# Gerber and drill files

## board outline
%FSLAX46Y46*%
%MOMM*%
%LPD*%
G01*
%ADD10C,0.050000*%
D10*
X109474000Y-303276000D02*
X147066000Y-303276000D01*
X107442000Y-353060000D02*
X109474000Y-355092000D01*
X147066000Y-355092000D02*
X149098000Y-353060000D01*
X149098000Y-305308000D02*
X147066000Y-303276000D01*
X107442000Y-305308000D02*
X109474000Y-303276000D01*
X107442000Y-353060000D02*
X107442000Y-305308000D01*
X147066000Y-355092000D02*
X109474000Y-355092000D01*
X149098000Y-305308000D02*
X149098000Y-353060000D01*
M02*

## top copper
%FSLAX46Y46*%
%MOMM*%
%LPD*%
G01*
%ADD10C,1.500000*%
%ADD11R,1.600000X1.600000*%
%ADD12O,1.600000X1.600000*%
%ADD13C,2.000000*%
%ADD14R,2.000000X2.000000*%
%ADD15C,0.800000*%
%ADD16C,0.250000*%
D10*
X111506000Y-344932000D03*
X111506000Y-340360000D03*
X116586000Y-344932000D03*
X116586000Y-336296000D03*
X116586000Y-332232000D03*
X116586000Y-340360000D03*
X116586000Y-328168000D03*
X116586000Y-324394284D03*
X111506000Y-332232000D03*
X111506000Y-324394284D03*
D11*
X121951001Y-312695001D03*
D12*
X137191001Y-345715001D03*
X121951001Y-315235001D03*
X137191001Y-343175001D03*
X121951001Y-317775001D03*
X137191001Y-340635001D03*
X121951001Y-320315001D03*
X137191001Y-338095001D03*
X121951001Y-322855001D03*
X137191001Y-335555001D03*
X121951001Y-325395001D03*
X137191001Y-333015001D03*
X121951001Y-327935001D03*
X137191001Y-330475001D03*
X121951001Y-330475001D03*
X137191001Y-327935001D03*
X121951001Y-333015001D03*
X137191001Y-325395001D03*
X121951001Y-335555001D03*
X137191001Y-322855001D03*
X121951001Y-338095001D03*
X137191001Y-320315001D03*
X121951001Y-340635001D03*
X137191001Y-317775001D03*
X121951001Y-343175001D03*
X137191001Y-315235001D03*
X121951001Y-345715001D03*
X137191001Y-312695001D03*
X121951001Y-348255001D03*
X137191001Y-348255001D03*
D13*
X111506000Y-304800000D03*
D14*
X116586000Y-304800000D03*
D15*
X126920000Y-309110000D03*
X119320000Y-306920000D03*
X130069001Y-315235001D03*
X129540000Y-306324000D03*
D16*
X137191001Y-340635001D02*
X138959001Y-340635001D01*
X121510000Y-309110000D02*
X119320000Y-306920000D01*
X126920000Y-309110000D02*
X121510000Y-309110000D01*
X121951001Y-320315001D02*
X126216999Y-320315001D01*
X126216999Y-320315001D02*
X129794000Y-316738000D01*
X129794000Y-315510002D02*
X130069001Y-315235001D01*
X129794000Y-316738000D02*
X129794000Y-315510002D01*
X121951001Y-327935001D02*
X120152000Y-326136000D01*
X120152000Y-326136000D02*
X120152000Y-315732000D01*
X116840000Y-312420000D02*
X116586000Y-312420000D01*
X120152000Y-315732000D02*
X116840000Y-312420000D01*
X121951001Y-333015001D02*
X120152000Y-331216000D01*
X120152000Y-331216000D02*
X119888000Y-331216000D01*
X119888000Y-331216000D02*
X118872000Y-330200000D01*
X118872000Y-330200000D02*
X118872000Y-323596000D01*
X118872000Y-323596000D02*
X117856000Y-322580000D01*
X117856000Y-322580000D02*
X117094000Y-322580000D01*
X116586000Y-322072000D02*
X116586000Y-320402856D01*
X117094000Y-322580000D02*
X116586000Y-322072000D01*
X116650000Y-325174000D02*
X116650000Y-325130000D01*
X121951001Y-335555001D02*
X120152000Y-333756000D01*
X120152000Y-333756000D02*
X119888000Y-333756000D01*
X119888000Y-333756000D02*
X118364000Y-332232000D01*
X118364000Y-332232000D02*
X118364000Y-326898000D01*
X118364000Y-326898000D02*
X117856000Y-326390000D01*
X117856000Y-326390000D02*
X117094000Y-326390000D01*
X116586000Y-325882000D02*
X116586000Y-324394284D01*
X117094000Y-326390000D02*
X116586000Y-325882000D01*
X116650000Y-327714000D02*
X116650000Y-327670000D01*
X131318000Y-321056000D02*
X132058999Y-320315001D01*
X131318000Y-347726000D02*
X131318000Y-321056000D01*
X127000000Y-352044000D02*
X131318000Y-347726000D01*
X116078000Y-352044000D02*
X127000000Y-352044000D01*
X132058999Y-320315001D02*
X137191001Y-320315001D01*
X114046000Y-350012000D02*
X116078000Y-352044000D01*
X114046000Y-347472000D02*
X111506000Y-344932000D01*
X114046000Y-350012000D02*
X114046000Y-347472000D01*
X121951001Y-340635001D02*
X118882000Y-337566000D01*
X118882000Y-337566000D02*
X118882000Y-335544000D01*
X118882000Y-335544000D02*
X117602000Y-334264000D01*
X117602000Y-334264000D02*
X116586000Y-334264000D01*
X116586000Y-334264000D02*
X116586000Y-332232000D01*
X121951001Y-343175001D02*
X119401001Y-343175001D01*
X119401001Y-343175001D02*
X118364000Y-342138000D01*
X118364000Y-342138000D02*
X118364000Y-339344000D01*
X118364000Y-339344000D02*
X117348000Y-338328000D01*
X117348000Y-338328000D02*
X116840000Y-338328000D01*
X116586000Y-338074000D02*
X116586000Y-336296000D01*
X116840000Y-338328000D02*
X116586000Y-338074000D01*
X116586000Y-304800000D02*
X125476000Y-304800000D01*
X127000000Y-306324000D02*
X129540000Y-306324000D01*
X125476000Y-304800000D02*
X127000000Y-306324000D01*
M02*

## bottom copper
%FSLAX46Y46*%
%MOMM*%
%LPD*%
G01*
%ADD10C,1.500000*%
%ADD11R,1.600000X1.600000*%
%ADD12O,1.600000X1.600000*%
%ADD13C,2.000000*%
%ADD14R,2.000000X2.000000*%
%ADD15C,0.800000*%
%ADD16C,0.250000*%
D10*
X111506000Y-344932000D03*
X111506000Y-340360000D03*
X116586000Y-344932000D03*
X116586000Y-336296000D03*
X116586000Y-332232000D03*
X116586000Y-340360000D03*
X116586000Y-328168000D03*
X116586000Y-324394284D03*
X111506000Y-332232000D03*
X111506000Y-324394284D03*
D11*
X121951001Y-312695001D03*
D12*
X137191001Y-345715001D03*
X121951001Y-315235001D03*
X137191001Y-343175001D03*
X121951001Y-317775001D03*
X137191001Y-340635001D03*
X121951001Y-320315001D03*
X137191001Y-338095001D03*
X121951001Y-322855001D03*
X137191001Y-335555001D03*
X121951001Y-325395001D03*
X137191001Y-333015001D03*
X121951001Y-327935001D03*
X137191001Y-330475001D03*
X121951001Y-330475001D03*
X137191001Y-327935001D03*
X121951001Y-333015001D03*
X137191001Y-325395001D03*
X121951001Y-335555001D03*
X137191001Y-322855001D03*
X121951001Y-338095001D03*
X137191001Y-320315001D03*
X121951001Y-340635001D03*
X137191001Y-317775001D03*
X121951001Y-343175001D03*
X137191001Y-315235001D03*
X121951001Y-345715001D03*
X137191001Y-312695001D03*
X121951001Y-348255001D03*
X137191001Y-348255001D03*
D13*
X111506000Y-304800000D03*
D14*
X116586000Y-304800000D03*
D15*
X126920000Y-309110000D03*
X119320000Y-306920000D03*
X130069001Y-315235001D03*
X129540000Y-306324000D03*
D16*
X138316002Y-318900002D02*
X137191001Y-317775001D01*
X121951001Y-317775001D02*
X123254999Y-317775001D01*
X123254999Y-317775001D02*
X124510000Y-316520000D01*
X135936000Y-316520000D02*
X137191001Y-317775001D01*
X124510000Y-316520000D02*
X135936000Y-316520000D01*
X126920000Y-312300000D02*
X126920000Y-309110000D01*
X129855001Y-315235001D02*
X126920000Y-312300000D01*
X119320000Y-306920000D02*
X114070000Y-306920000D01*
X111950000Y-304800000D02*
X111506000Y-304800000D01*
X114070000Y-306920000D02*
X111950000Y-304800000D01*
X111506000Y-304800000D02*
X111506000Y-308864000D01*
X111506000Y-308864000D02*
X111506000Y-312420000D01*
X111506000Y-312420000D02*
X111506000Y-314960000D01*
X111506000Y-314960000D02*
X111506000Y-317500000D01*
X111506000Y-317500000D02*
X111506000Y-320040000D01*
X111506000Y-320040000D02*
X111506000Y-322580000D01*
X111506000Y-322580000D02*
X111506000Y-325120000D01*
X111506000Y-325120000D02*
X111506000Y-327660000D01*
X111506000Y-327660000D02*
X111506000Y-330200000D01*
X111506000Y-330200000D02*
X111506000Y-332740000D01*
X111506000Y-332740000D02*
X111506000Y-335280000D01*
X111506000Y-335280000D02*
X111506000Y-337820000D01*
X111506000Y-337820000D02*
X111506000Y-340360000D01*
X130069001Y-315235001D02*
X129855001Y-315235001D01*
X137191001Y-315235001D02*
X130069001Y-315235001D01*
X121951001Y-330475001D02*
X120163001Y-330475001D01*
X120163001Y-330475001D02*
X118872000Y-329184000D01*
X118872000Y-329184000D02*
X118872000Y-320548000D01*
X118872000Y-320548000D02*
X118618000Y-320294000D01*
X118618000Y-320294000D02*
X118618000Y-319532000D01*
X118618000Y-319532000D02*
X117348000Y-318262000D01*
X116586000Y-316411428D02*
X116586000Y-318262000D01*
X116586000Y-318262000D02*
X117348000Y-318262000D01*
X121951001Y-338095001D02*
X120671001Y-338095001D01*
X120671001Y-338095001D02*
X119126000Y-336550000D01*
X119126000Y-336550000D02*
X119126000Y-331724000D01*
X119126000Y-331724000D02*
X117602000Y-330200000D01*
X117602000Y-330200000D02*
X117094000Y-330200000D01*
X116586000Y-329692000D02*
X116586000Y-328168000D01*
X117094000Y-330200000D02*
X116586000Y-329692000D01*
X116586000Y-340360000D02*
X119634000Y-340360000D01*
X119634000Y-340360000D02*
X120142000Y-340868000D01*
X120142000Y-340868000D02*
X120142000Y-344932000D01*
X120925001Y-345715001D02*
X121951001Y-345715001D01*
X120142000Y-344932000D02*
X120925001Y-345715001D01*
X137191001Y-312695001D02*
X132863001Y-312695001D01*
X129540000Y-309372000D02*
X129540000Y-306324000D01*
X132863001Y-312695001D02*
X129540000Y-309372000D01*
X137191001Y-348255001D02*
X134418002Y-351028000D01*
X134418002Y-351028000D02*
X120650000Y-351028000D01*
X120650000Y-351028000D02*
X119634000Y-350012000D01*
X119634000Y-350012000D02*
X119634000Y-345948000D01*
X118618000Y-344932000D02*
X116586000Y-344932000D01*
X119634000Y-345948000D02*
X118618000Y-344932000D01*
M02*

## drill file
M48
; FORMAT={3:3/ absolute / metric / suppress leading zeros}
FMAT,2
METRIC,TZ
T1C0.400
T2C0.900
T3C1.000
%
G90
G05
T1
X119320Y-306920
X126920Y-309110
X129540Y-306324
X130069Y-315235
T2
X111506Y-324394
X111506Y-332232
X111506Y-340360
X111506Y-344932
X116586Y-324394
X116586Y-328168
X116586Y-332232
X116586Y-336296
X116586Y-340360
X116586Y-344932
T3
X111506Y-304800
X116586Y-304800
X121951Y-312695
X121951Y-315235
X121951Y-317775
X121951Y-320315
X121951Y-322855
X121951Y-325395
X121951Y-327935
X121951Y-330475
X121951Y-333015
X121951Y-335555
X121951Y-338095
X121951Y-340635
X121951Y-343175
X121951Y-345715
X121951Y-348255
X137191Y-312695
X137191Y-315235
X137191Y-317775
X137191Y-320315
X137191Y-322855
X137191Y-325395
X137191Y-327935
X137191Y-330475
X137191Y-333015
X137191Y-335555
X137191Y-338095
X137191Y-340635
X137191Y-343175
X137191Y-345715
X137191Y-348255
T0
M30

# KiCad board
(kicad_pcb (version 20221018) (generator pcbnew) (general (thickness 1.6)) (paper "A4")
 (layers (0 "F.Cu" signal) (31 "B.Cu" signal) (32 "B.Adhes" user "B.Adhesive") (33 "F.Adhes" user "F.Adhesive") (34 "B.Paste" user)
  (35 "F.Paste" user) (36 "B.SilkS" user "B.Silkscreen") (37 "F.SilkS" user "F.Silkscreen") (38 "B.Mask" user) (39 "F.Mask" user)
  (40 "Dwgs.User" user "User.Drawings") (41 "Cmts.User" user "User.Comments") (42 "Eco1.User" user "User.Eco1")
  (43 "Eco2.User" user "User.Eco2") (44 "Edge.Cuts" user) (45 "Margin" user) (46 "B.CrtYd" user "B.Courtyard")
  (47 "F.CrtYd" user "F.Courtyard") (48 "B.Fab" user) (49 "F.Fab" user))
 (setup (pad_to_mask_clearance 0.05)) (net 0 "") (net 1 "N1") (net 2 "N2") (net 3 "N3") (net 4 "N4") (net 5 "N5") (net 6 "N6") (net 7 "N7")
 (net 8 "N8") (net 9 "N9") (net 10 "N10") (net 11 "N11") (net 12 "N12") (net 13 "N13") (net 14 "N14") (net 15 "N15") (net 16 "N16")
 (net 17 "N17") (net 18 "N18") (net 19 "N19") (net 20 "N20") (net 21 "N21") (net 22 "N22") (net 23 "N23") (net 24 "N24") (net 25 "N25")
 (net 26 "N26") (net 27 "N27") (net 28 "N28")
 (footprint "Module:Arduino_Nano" (layer "F.Cu") (at 121.951001 312.695001)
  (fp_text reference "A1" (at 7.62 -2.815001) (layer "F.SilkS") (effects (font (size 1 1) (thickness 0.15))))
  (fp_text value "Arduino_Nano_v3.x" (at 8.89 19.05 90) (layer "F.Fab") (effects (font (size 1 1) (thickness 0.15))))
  (pad "1" thru_hole rect (at 0 0) (size 1.6 1.6) (drill 1) (layers "*.Cu" "*.Mask") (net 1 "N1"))
  (pad "2" thru_hole oval (at 0 2.54) (size 1.6 1.6) (drill 1) (layers "*.Cu" "*.Mask") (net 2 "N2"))
  (pad "3" thru_hole oval (at 0 5.08) (size 1.6 1.6) (drill 1) (layers "*.Cu" "*.Mask") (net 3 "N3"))
  (pad "4" thru_hole oval (at 0 7.62) (size 1.6 1.6) (drill 1) (layers "*.Cu" "*.Mask") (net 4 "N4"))
  (pad "5" thru_hole oval (at 0 10.16) (size 1.6 1.6) (drill 1) (layers "*.Cu" "*.Mask") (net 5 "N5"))
  (pad "6" thru_hole oval (at 0 12.7) (size 1.6 1.6) (drill 1) (layers "*.Cu" "*.Mask") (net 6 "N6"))
  (pad "7" thru_hole oval (at 0 15.24) (size 1.6 1.6) (drill 1) (layers "*.Cu" "*.Mask") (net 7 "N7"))
  (pad "8" thru_hole oval (at 0 17.78) (size 1.6 1.6) (drill 1) (layers "*.Cu" "*.Mask") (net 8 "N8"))
  (pad "9" thru_hole oval (at 0 20.32) (size 1.6 1.6) (drill 1) (layers "*.Cu" "*.Mask") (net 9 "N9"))
  (pad "10" thru_hole oval (at 0 22.86) (size 1.6 1.6) (drill 1) (layers "*.Cu" "*.Mask") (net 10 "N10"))
  (pad "11" thru_hole oval (at 0 25.4) (size 1.6 1.6) (drill 1) (layers "*.Cu" "*.Mask") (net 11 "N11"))
  (pad "12" thru_hole oval (at 0 27.94) (size 1.6 1.6) (drill 1) (layers "*.Cu" "*.Mask") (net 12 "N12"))
  (pad "13" thru_hole oval (at 0 30.48) (size 1.6 1.6) (drill 1) (layers "*.Cu" "*.Mask") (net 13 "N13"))
  (pad "14" thru_hole oval (at 0 33.02) (size 1.6 1.6) (drill 1) (layers "*.Cu" "*.Mask") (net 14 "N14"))
  (pad "15" thru_hole oval (at 0 35.56) (size 1.6 1.6) (drill 1) (layers "*.Cu" "*.Mask") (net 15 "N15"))
  (pad "16" thru_hole oval (at 15.24 35.56) (size 1.6 1.6) (drill 1) (layers "*.Cu" "*.Mask") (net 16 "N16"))
  (pad "17" thru_hole oval (at 15.24 33.02) (size 1.6 1.6) (drill 1) (layers "*.Cu" "*.Mask") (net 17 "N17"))
  (pad "18" thru_hole oval (at 15.24 30.48) (size 1.6 1.6) (drill 1) (layers "*.Cu" "*.Mask") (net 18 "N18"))
  (pad "19" thru_hole oval (at 15.24 27.94) (size 1.6 1.6) (drill 1) (layers "*.Cu" "*.Mask") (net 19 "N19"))
  (pad "20" thru_hole oval (at 15.24 25.4) (size 1.6 1.6) (drill 1) (layers "*.Cu" "*.Mask") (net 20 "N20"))
  (pad "21" thru_hole oval (at 15.24 22.86) (size 1.6 1.6) (drill 1) (layers "*.Cu" "*.Mask") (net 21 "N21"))
  (pad "22" thru_hole oval (at 15.24 20.32) (size 1.6 1.6) (drill 1) (layers "*.Cu" "*.Mask") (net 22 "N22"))
  (pad "23" thru_hole oval (at 15.24 17.78) (size 1.6 1.6) (drill 1) (layers "*.Cu" "*.Mask") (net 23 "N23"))
  (pad "24" thru_hole oval (at 15.24 15.24) (size 1.6 1.6) (drill 1) (layers "*.Cu" "*.Mask") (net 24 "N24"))
  (pad "25" thru_hole oval (at 15.24 12.7) (size 1.6 1.6) (drill 1) (layers "*.Cu" "*.Mask") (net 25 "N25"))
  (pad "26" thru_hole oval (at 15.24 10.16) (size 1.6 1.6) (drill 1) (layers "*.Cu" "*.Mask") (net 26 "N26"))
  (pad "27" thru_hole oval (at 15.24 7.62) (size 1.6 1.6) (drill 1) (layers "*.Cu" "*.Mask") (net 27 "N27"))
  (pad "28" thru_hole oval (at 15.24 5.08) (size 1.6 1.6) (drill 1) (layers "*.Cu" "*.Mask") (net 3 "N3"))
  (pad "29" thru_hole oval (at 15.24 2.54) (size 1.6 1.6) (drill 1) (layers "*.Cu" "*.Mask") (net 4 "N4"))
  (pad "30" thru_hole oval (at 15.24 0) (size 1.6 1.6) (drill 1) (layers "*.Cu" "*.Mask") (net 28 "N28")))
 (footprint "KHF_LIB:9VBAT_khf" (layer "F.Cu") (at 111.506 304.8)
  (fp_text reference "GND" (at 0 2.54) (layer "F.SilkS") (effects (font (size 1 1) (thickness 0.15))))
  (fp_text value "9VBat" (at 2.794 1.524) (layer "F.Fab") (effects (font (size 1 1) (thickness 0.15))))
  (pad "1" thru_hole circle (at 0 0) (size 2 2) (drill 1) (layers "*.Cu" "*.Mask") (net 4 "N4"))
  (pad "2" thru_hole rect (at 5.08 0) (size 2 2) (drill 1) (layers "*.Cu" "*.Mask") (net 28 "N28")))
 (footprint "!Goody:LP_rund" (layer "F.Cu") (at 116.586 336.296)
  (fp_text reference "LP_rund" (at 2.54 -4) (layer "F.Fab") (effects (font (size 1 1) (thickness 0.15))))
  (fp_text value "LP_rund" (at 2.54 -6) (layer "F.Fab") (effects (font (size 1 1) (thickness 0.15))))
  (pad "1" thru_hole circle (at 0 0) (size 1.5 1.5) (drill 0.9) (layers "*.Cu" "*.Mask") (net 13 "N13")))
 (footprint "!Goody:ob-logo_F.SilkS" (layer "F.Cu") (at 130.048 329.692 90)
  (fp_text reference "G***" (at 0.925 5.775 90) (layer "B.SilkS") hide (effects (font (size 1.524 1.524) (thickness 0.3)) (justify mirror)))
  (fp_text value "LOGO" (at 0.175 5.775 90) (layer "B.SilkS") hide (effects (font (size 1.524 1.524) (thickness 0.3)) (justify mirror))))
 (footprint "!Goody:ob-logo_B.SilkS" (layer "F.Cu") (at 146.05 323.596 90)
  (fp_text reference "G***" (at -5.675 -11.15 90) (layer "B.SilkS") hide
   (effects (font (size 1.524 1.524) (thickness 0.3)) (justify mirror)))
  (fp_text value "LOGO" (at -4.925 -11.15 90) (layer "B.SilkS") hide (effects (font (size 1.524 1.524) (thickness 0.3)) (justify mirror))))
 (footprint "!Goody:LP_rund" (layer "F.Cu") (at 116.586 344.932)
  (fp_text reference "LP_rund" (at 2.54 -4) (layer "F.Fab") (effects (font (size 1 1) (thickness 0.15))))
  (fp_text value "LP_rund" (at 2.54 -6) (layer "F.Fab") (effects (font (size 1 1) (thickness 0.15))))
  (pad "1" thru_hole circle (at 0 0) (size 1.5 1.5) (drill 0.9) (layers "*.Cu" "*.Mask") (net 16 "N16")))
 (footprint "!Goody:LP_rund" (layer "F.Cu") (at 111.506 340.36)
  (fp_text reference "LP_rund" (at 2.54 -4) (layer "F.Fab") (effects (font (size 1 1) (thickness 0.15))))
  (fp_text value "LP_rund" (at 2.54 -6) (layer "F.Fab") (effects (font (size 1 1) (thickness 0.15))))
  (pad "1" thru_hole circle (at 0 0) (size 1.5 1.5) (drill 0.9) (layers "*.Cu" "*.Mask") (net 4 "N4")))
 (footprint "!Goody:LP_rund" (layer "F.Cu") (at 111.506 344.932)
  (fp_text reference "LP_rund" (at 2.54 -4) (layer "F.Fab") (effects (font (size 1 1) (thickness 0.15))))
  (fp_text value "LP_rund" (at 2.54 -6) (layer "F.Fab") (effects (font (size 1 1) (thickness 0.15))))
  (pad "1" thru_hole circle (at 0 0) (size 1.5 1.5) (drill 0.9) (layers "*.Cu" "*.Mask") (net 27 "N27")))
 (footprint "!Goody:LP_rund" (layer "F.Cu") (at 116.586 324.394284)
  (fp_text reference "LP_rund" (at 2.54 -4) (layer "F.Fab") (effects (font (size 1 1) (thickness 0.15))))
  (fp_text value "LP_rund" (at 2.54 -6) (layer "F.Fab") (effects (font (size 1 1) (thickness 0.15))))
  (pad "1" thru_hole circle (at 0 0) (size 1.5 1.5) (drill 0.9) (layers "*.Cu" "*.Mask") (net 10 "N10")))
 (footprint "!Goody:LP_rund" (layer "F.Cu") (at 111.506 330.2)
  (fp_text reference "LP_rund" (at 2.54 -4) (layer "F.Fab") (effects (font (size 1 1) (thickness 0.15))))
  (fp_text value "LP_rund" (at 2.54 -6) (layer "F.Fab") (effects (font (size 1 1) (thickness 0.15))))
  (pad "1" thru_hole circle (at 0 -5.805716) (size 1.5 1.5) (drill 0.9) (layers "*.Cu" "*.Mask") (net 4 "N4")))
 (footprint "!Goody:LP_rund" (layer "F.Cu") (at 116.586 328.168)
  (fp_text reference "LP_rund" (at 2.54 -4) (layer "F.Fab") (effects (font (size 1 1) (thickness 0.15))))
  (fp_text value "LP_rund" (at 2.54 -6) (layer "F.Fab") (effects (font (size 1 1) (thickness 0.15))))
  (pad "1" thru_hole circle (at 0 0) (size 1.5 1.5) (drill 0.9) (layers "*.Cu" "*.Mask") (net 11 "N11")))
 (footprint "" (layer "F.Cu") (at 112.268 348.488)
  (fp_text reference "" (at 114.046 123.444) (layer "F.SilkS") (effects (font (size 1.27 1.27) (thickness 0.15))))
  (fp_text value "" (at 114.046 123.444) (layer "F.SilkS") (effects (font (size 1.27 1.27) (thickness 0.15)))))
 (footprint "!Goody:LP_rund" (layer "F.Cu") (at 111.506 335.13486)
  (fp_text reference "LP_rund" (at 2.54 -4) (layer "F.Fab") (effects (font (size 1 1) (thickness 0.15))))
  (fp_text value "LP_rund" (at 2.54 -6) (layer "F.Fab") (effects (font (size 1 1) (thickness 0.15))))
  (pad "1" thru_hole circle (at 0 -2.90286) (size 1.5 1.5) (drill 0.9) (layers "*.Cu" "*.Mask") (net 4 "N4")))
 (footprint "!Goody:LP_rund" (layer "F.Cu") (at 116.586 340.36)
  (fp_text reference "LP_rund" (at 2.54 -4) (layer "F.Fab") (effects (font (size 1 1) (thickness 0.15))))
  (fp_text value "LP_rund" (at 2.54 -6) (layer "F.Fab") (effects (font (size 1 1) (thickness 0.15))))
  (pad "1" thru_hole circle (at 0 0) (size 1.5 1.5) (drill 0.9) (layers "*.Cu" "*.Mask") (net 14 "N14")))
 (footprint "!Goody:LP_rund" (layer "F.Cu") (at 116.586 332.232)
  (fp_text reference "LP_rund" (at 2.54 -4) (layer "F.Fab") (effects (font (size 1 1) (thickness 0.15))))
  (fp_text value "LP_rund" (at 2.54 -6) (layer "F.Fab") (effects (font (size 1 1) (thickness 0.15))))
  (pad "1" thru_hole circle (at 0 0) (size 1.5 1.5) (drill 0.9) (layers "*.Cu" "*.Mask") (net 12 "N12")))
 (gr_line (start 107.442 353.06) (end 107.442 305.308) (stroke (width 0.05) (type solid)) (layer "Edge.Cuts"))
 (gr_line (start 109.474 303.276) (end 147.066 303.276) (stroke (width 0.05) (type solid)) (layer "Edge.Cuts"))
 (gr_line (start 107.442 305.308) (end 109.474 303.276) (stroke (width 0.05) (type solid)) (layer "Edge.Cuts"))
 (gr_line (start 147.066 355.092) (end 149.098 353.06) (stroke (width 0.05) (type solid)) (layer "Edge.Cuts"))
 (gr_line (start 147.066 355.092) (end 109.474 355.092) (stroke (width 0.05) (type solid)) (layer "Edge.Cuts"))
 (gr_line (start 149.098 305.308) (end 147.066 303.276) (stroke (width 0.05) (type solid)) (layer "Edge.Cuts"))
 (gr_line (start 149.098 305.308) (end 149.098 353.06) (stroke (width 0.05) (type solid)) (layer "Edge.Cuts"))
 (gr_line (start 107.442 353.06) (end 109.474 355.092) (stroke (width 0.05) (type solid)) (layer "Edge.Cuts"))
 (segment (start 138.316002 318.900002) (end 137.191001 317.775001) (width 0.25) (layer "B.Cu") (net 3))
 (segment (start 121.951001 317.775001) (end 123.254999 317.775001) (width 0.25) (layer "B.Cu") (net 3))
 (segment (start 135.936 316.52) (end 137.191001 317.775001) (width 0.25) (layer "B.Cu") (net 3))
 (segment (start 123.254999 317.775001) (end 124.51 316.52) (width 0.25) (layer "B.Cu") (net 3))
 (segment (start 124.51 316.52) (end 135.936 316.52) (width 0.25) (layer "B.Cu") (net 3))
 (segment (start 137.191001 340.635001) (end 138.959001 340.635001) (width 0.25) (layer "F.Cu") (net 19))
 (segment (start 129.794 315.510002) (end 130.069001 315.235001) (width 0.25) (layer "F.Cu") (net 4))
 (segment (start 121.51 309.11) (end 119.32 306.92) (width 0.25) (layer "F.Cu") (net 4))
 (segment (start 129.794 316.738) (end 129.794 315.510002) (width 0.25) (layer "F.Cu") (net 4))
 (segment (start 126.216999 320.315001) (end 129.794 316.738) (width 0.25) (layer "F.Cu") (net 4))
 (segment (start 126.92 309.11) (end 121.51 309.11) (width 0.25) (layer "F.Cu") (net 4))
 (segment (start 121.951001 320.315001) (end 126.216999 320.315001) (width 0.25) (layer "F.Cu") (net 4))
 (via (at 126.92 309.11) (size 0.8) (drill 0.4) (layers "F.Cu" "B.Cu") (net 4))
 (via (at 130.069001 315.235001) (size 0.8) (drill 0.4) (layers "F.Cu" "B.Cu") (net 4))
 (via (at 119.32 306.92) (size 0.8) (drill 0.4) (layers "F.Cu" "B.Cu") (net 4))
 (segment (start 111.95 304.8) (end 111.506 304.8) (width 0.25) (layer "B.Cu") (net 4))
 (segment (start 111.506 330.2) (end 111.506 332.74) (width 0.25) (layer "B.Cu") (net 4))
 (segment (start 111.506 325.12) (end 111.506 327.66) (width 0.25) (layer "B.Cu") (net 4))
 (segment (start 111.506 312.42) (end 111.506 314.96) (width 0.25) (layer "B.Cu") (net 4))
 (segment (start 111.506 335.28) (end 111.506 337.82) (width 0.25) (layer "B.Cu") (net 4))
 (segment (start 111.506 332.74) (end 111.506 335.28) (width 0.25) (layer "B.Cu") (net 4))
 (segment (start 111.506 327.66) (end 111.506 330.2) (width 0.25) (layer "B.Cu") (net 4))
 (segment (start 137.191001 315.235001) (end 130.069001 315.235001) (width 0.25) (layer "B.Cu") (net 4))
 (segment (start 111.506 308.864) (end 111.506 312.42) (width 0.25) (layer "B.Cu") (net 4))
 (segment (start 111.506 320.04) (end 111.506 322.58) (width 0.25) (layer "B.Cu") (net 4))
 (segment (start 130.069001 315.235001) (end 129.855001 315.235001) (width 0.25) (layer "B.Cu") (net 4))
 (segment (start 111.506 337.82) (end 111.506 340.36) (width 0.25) (layer "B.Cu") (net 4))
 (segment (start 111.506 304.8) (end 111.506 308.864) (width 0.25) (layer "B.Cu") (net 4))
 (segment (start 111.506 322.58) (end 111.506 325.12) (width 0.25) (layer "B.Cu") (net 4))
 (segment (start 114.07 306.92) (end 111.95 304.8) (width 0.25) (layer "B.Cu") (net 4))
 (segment (start 119.32 306.92) (end 114.07 306.92) (width 0.25) (layer "B.Cu") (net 4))
 (segment (start 126.92 312.3) (end 126.92 309.11) (width 0.25) (layer "B.Cu") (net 4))
 (segment (start 111.506 314.96) (end 111.506 317.5) (width 0.25) (layer "B.Cu") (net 4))
 (segment (start 111.506 317.5) (end 111.506 320.04) (width 0.25) (layer "B.Cu") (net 4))
 (segment (start 129.855001 315.235001) (end 126.92 312.3) (width 0.25) (layer "B.Cu") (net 4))
 (segment (start 120.152 326.136) (end 120.152 315.732) (width 0.25) (layer "F.Cu") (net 7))
 (segment (start 121.951001 327.935001) (end 120.152 326.136) (width 0.25) (layer "F.Cu") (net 7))
 (segment (start 120.152 315.732) (end 116.84 312.42) (width 0.25) (layer "F.Cu") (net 7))
 (segment (start 116.84 312.42) (end 116.586 312.42) (width 0.25) (layer "F.Cu") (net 7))
 (segment (start 118.618 319.532) (end 117.348 318.262) (width 0.25) (layer "B.Cu") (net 8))
 (segment (start 118.872 329.184) (end 118.872 320.548) (width 0.25) (layer "B.Cu") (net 8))
 (segment (start 121.951001 330.475001) (end 120.163001 330.475001) (width 0.25) (layer "B.Cu") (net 8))
 (segment (start 120.163001 330.475001) (end 118.872 329.184) (width 0.25) (layer "B.Cu") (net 8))
 (segment (start 116.586 316.411428) (end 116.586 318.262) (width 0.25) (layer "B.Cu") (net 8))
 (segment (start 116.586 318.262) (end 117.348 318.262) (width 0.25) (layer "B.Cu") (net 8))
 (segment (start 118.618 320.294) (end 118.618 319.532) (width 0.25) (layer "B.Cu") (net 8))
 (segment (start 118.872 320.548) (end 118.618 320.294) (width 0.25) (layer "B.Cu") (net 8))
 (segment (start 119.888 331.216) (end 118.872 330.2) (width 0.25) (layer "F.Cu") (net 9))
 (segment (start 117.856 322.58) (end 117.094 322.58) (width 0.25) (layer "F.Cu") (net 9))
 (segment (start 118.872 323.596) (end 117.856 322.58) (width 0.25) (layer "F.Cu") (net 9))
 (segment (start 118.872 330.2) (end 118.872 323.596) (width 0.25) (layer "F.Cu") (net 9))
 (segment (start 117.094 322.58) (end 116.586 322.072) (width 0.25) (layer "F.Cu") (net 9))
 (segment (start 120.152 331.216) (end 119.888 331.216) (width 0.25) (layer "F.Cu") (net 9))
 (segment (start 116.586 322.072) (end 116.586 320.402856) (width 0.25) (layer "F.Cu") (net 9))
 (segment (start 121.951001 333.015001) (end 120.152 331.216) (width 0.25) (layer "F.Cu") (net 9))
 (segment (start 120.152 333.756) (end 119.888 333.756) (width 0.25) (layer "F.Cu") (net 10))
 (segment (start 118.364 332.232) (end 118.364 326.898) (width 0.25) (layer "F.Cu") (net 10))
 (segment (start 117.856 326.39) (end 117.094 326.39) (width 0.25) (layer "F.Cu") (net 10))
 (segment (start 121.951001 335.555001) (end 120.152 333.756) (width 0.25) (layer "F.Cu") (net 10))
 (segment (start 119.888 333.756) (end 118.364 332.232) (width 0.25) (layer "F.Cu") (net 10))
 (segment (start 116.65 325.174) (end 116.65 325.13) (width 0.25) (layer "F.Cu") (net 10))
 (segment (start 117.094 326.39) (end 116.586 325.882) (width 0.25) (layer "F.Cu") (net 10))
 (segment (start 118.364 326.898) (end 117.856 326.39) (width 0.25) (layer "F.Cu") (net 10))
 (segment (start 116.586 325.882) (end 116.586 324.394284) (width 0.25) (layer "F.Cu") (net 10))
 (segment (start 116.65 327.714) (end 116.65 327.67) (width 0.25) (layer "F.Cu") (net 11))
 (segment (start 121.951001 338.095001) (end 120.671001 338.095001) (width 0.25) (layer "B.Cu") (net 11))
 (segment (start 119.126 336.55) (end 119.126 331.724) (width 0.25) (layer "B.Cu") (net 11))
 (segment (start 116.586 329.692) (end 116.586 328.168) (width 0.25) (layer "B.Cu") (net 11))
 (segment (start 117.094 330.2) (end 116.586 329.692) (width 0.25) (layer "B.Cu") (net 11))
 (segment (start 120.671001 338.095001) (end 119.126 336.55) (width 0.25) (layer "B.Cu") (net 11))
 (segment (start 117.602 330.2) (end 117.094 330.2) (width 0.25) (layer "B.Cu") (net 11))
 (segment (start 119.126 331.724) (end 117.602 330.2) (width 0.25) (layer "B.Cu") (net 11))
 (segment (start 116.078 352.044) (end 127 352.044) (width 0.25) (layer "F.Cu") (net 27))
 (segment (start 127 352.044) (end 131.318 347.726) (width 0.25) (layer "F.Cu") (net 27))
 (segment (start 131.318 321.056) (end 132.058999 320.315001) (width 0.25) (layer "F.Cu") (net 27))
 (segment (start 132.058999 320.315001) (end 137.191001 320.315001) (width 0.25) (layer "F.Cu") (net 27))
 (segment (start 114.046 350.012) (end 116.078 352.044) (width 0.25) (layer "F.Cu") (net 27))
 (segment (start 131.318 347.726) (end 131.318 321.056) (width 0.25) (layer "F.Cu") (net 27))
 (segment (start 114.046 347.472) (end 111.506 344.932) (width 0.25) (layer "F.Cu") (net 27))
 (segment (start 114.046 350.012) (end 114.046 347.472) (width 0.25) (layer "F.Cu") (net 27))
 (segment (start 118.882 335.544) (end 117.602 334.264) (width 0.25) (layer "F.Cu") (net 12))
 (segment (start 118.882 337.566) (end 118.882 335.544) (width 0.25) (layer "F.Cu") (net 12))
 (segment (start 121.951001 340.635001) (end 118.882 337.566) (width 0.25) (layer "F.Cu") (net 12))
 (segment (start 116.586 334.264) (end 116.586 332.232) (width 0.25) (layer "F.Cu") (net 12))
 (segment (start 117.602 334.264) (end 116.586 334.264) (width 0.25) (layer "F.Cu") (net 12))
 (segment (start 121.951001 343.175001) (end 119.401001 343.175001) (width 0.25) (layer "F.Cu") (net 13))
 (segment (start 119.401001 343.175001) (end 118.364 342.138) (width 0.25) (layer "F.Cu") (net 13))
 (segment (start 116.84 338.328) (end 116.586 338.074) (width 0.25) (layer "F.Cu") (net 13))
 (segment (start 118.364 339.344) (end 117.348 338.328) (width 0.25) (layer "F.Cu") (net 13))
 (segment (start 118.364 342.138) (end 118.364 339.344) (width 0.25) (layer "F.Cu") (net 13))
 (segment (start 116.586 338.074) (end 116.586 336.296) (width 0.25) (layer "F.Cu") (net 13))
 (segment (start 117.348 338.328) (end 116.84 338.328) (width 0.25) (layer "F.Cu") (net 13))
 (segment (start 120.925001 345.715001) (end 121.951001 345.715001) (width 0.25) (layer "B.Cu") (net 14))
 (segment (start 120.142 340.868) (end 120.142 344.932) (width 0.25) (layer "B.Cu") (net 14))
 (segment (start 120.142 344.932) (end 120.925001 345.715001) (width 0.25) (layer "B.Cu") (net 14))
 (segment (start 116.586 340.36) (end 119.634 340.36) (width 0.25) (layer "B.Cu") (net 14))
 (segment (start 119.634 340.36) (end 120.142 340.868) (width 0.25) (layer "B.Cu") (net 14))
 (segment (start 127 306.324) (end 129.54 306.324) (width 0.25) (layer "F.Cu") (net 28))
 (segment (start 125.476 304.8) (end 127 306.324) (width 0.25) (layer "F.Cu") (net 28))
 (segment (start 116.586 304.8) (end 125.476 304.8) (width 0.25) (layer "F.Cu") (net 28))
 (via (at 129.54 306.324) (size 0.8) (drill 0.4) (layers "F.Cu" "B.Cu") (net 28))
 (segment (start 129.54 309.372) (end 129.54 306.324) (width 0.25) (layer "B.Cu") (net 28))
 (segment (start 132.863001 312.695001) (end 129.54 309.372) (width 0.25) (layer "B.Cu") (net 28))
 (segment (start 137.191001 312.695001) (end 132.863001 312.695001) (width 0.25) (layer "B.Cu") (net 28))
 (segment (start 120.65 351.028) (end 119.634 350.012) (width 0.25) (layer "B.Cu") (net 16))
 (segment (start 134.418002 351.028) (end 120.65 351.028) (width 0.25) (layer "B.Cu") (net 16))
 (segment (start 119.634 350.012) (end 119.634 345.948) (width 0.25) (layer "B.Cu") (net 16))
 (segment (start 119.634 345.948) (end 118.618 344.932) (width 0.25) (layer "B.Cu") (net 16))
 (segment (start 137.191001 348.255001) (end 134.418002 351.028) (width 0.25) (layer "B.Cu") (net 16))
 (segment (start 118.618 344.932) (end 116.586 344.932) (width 0.25) (layer "B.Cu") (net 16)))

